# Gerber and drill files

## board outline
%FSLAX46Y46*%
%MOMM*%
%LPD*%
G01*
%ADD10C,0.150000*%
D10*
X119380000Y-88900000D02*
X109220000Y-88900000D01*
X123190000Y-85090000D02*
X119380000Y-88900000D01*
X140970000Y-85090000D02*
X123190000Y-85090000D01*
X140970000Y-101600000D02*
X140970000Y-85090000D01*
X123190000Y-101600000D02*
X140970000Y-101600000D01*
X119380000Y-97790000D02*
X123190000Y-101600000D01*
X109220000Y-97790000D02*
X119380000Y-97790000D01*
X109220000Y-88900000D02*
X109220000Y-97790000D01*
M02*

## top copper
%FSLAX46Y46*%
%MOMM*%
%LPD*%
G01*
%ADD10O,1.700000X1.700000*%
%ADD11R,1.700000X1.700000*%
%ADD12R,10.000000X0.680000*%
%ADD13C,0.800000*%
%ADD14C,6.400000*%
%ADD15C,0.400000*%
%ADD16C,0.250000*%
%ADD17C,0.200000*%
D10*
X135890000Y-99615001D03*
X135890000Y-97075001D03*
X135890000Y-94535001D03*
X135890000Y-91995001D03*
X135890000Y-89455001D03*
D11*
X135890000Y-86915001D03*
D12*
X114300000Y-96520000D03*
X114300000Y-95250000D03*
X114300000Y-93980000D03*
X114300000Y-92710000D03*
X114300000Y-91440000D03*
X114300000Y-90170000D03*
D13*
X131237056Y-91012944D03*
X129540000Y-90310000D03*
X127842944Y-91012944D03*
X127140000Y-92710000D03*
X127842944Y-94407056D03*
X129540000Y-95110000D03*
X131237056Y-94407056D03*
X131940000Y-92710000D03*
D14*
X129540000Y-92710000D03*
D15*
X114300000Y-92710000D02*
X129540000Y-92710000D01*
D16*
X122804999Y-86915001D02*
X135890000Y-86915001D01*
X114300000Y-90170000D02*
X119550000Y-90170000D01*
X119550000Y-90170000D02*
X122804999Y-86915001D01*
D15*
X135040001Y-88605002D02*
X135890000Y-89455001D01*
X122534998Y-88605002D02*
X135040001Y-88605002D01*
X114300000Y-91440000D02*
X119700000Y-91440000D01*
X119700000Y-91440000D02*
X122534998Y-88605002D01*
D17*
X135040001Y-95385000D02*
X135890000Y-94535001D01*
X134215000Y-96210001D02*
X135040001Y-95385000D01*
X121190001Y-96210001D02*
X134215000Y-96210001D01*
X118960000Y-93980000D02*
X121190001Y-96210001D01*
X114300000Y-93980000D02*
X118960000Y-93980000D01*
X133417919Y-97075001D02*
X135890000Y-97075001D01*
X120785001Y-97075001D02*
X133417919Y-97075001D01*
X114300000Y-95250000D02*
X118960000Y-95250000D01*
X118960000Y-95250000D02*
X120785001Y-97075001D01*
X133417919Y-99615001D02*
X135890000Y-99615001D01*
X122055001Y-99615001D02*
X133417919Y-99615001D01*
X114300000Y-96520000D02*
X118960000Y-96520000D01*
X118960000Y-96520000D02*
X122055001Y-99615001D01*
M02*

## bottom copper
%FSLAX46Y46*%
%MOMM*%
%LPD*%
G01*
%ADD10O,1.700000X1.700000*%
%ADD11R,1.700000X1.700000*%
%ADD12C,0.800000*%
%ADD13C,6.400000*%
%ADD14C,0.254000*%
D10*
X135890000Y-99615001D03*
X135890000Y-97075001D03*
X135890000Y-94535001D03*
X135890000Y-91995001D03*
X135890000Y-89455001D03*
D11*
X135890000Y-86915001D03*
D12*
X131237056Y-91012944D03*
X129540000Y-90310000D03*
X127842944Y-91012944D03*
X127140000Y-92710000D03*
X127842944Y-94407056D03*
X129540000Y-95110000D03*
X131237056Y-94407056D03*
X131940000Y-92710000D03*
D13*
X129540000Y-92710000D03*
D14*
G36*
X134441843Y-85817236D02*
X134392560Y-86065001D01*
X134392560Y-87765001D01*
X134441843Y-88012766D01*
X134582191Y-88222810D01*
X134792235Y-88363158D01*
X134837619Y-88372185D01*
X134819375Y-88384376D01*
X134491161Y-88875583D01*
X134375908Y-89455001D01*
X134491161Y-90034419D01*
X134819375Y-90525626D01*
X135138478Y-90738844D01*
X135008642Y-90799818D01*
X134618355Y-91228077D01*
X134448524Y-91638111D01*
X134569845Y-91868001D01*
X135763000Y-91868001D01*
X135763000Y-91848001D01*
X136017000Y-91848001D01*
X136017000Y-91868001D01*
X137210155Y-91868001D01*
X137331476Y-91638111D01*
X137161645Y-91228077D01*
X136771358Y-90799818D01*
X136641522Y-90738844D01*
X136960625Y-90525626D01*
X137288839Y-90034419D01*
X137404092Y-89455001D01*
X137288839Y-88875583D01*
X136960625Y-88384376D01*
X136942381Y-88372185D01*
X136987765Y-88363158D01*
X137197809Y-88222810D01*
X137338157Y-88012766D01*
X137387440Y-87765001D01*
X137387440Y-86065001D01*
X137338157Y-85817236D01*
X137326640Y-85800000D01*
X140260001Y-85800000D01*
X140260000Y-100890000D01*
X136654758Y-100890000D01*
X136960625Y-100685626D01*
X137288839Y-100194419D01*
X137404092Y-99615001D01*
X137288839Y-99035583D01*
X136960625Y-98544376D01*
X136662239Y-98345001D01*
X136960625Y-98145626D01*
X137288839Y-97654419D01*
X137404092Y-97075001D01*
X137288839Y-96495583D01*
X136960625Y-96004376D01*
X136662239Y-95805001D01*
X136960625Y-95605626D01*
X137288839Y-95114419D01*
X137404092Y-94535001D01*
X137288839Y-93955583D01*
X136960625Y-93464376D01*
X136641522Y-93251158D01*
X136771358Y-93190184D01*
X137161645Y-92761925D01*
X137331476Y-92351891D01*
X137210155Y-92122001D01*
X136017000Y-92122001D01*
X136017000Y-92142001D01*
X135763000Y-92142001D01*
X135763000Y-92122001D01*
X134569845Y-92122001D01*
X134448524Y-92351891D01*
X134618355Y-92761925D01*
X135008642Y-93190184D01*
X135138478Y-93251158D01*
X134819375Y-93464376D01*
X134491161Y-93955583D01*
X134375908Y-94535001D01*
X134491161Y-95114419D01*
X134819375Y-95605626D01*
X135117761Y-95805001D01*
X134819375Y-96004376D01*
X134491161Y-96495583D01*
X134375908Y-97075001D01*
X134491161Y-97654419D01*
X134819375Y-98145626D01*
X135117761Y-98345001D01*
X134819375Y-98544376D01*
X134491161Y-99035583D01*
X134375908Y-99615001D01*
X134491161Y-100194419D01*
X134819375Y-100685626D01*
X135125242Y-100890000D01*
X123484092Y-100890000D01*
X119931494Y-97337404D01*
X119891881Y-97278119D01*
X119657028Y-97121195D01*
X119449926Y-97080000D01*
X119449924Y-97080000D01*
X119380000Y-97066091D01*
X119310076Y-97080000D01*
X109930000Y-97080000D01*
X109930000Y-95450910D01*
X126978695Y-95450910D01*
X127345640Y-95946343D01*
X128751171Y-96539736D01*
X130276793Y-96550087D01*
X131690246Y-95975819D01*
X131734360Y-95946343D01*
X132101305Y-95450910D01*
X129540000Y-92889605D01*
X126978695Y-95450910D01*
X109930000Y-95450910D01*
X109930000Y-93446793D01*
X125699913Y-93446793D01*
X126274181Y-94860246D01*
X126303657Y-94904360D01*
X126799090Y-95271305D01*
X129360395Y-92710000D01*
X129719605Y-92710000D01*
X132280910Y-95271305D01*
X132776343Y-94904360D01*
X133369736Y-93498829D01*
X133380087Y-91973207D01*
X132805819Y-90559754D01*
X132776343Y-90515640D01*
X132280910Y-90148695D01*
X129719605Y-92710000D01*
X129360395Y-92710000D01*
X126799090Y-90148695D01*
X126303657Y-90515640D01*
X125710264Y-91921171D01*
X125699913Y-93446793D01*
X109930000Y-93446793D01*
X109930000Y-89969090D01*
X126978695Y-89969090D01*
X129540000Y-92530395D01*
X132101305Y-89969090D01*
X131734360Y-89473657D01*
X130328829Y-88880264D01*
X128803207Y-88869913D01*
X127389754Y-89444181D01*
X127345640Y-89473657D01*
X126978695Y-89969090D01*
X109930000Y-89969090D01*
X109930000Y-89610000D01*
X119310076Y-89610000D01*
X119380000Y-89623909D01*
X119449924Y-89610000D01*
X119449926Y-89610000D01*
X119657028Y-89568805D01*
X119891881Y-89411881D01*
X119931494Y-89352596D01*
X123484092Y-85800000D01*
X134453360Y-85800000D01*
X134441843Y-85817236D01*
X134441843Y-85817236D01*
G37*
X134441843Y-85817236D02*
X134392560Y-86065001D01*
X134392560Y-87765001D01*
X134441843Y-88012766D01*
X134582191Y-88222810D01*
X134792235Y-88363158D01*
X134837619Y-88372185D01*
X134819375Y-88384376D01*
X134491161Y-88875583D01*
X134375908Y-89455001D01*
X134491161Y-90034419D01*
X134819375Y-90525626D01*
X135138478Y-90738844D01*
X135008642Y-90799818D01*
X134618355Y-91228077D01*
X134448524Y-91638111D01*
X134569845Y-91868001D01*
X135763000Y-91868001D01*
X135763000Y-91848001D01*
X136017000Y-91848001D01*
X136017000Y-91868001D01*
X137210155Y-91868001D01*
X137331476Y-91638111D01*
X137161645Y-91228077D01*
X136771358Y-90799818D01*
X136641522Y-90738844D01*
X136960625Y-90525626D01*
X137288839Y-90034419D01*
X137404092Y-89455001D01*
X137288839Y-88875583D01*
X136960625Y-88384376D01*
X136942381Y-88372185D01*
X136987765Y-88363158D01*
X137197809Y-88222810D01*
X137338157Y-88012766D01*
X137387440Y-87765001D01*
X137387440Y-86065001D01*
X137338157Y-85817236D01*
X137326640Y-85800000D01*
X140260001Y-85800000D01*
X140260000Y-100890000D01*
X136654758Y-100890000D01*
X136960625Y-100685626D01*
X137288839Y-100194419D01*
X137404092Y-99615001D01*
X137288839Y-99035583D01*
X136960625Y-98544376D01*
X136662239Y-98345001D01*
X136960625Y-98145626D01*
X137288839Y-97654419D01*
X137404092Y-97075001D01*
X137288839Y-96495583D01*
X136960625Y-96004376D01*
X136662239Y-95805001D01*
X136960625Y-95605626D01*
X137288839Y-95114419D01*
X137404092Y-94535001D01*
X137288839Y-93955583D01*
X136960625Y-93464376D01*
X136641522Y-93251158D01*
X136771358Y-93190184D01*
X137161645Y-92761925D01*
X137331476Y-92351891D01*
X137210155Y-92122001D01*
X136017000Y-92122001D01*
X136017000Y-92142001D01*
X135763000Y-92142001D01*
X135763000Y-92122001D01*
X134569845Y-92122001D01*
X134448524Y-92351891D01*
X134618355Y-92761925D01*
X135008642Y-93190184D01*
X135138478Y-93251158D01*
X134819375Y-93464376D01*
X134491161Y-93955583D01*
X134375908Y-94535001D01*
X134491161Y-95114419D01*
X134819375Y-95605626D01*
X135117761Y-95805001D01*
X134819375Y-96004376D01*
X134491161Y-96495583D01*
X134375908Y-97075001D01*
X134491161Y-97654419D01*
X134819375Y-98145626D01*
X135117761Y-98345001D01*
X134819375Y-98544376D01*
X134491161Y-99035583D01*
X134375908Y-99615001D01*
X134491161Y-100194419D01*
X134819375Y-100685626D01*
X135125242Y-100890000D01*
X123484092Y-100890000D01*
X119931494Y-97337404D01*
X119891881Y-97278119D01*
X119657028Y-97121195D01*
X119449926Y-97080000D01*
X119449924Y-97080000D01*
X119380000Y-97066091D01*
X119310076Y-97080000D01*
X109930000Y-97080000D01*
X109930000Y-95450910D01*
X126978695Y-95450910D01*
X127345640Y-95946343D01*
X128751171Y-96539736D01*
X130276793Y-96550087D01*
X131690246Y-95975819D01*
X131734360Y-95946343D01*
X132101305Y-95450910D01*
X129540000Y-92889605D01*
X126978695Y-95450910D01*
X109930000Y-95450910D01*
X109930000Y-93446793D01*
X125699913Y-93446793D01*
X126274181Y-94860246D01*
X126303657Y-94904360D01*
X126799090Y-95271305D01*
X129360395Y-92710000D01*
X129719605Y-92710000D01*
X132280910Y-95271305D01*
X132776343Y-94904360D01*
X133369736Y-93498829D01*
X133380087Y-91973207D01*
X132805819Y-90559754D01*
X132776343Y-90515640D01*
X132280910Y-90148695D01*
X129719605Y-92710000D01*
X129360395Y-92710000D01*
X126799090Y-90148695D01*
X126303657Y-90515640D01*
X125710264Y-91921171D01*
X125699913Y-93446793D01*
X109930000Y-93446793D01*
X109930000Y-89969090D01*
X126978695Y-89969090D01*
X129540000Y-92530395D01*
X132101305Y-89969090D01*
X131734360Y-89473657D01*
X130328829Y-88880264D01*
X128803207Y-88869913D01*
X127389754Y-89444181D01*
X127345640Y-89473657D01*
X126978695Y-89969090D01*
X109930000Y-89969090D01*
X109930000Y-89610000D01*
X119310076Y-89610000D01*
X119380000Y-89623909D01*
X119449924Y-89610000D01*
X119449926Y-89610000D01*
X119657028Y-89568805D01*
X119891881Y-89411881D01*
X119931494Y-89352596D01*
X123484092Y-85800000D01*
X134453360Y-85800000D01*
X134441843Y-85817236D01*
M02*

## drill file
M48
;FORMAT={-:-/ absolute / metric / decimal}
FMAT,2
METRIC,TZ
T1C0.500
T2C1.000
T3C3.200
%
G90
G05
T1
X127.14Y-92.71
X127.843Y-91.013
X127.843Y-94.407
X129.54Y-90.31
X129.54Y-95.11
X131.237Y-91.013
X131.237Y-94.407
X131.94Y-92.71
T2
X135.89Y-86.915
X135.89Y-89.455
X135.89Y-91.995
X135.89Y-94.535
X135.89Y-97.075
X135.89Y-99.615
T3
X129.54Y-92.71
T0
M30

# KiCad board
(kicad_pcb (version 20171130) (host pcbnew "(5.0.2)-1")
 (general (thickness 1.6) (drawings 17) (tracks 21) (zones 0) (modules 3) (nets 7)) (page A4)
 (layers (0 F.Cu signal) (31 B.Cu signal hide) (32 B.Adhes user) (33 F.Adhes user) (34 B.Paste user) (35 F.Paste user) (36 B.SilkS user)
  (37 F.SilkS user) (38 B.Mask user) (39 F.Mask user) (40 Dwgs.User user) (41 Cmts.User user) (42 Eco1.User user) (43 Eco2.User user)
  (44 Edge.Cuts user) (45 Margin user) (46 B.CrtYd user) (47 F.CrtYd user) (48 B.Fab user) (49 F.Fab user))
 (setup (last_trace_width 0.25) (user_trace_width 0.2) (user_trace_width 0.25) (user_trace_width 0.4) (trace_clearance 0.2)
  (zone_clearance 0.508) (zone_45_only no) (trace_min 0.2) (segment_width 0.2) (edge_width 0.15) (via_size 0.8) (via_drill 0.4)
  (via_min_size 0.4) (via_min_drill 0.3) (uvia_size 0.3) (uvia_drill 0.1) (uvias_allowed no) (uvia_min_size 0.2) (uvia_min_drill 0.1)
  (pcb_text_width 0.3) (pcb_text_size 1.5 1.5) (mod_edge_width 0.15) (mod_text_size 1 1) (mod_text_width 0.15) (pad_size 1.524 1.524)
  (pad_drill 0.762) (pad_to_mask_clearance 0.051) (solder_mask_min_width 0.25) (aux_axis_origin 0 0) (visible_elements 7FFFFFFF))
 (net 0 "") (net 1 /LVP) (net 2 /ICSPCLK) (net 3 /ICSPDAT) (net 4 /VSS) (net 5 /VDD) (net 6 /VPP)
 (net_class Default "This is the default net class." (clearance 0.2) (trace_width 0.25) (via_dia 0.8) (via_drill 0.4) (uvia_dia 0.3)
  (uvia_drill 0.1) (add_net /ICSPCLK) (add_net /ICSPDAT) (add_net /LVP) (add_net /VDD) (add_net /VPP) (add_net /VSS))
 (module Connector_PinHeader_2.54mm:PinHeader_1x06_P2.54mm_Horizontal (layer F.Cu) (at 135.89 86.915001)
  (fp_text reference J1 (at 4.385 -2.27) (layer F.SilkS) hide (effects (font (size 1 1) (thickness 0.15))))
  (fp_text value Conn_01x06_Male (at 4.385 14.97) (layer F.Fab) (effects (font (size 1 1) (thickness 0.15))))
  (pad 6 thru_hole oval (at 0 12.7) (size 1.7 1.7) (drill 1) (layers *.Cu *.Mask) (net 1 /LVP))
  (pad 5 thru_hole oval (at 0 10.16) (size 1.7 1.7) (drill 1) (layers *.Cu *.Mask) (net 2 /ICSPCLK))
  (pad 4 thru_hole oval (at 0 7.62) (size 1.7 1.7) (drill 1) (layers *.Cu *.Mask) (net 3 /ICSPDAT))
  (pad 3 thru_hole oval (at 0 5.08) (size 1.7 1.7) (drill 1) (layers *.Cu *.Mask) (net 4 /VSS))
  (pad 2 thru_hole oval (at 0 2.54) (size 1.7 1.7) (drill 1) (layers *.Cu *.Mask) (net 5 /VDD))
  (pad 1 thru_hole rect (at 0 0) (size 1.7 1.7) (drill 1) (layers *.Cu *.Mask) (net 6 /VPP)))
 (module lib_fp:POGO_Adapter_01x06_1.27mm (layer F.Cu) (at 114.3 93.98 270)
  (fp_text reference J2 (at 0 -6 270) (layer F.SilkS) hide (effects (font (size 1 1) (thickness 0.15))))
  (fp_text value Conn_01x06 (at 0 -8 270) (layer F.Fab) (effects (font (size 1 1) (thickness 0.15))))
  (pad 6 smd rect (at 2.54 0 270) (size 0.68 10) (layers F.Cu F.Paste F.Mask) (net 1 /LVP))
  (pad 5 smd rect (at 1.27 0 270) (size 0.68 10) (layers F.Cu F.Paste F.Mask) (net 2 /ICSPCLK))
  (pad 4 smd rect (at 0 0 270) (size 0.68 10) (layers F.Cu F.Paste F.Mask) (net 3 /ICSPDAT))
  (pad 3 smd rect (at -1.27 0 270) (size 0.68 10) (layers F.Cu F.Paste F.Mask) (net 4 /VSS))
  (pad 2 smd rect (at -2.54 0 270) (size 0.68 10) (layers F.Cu F.Paste F.Mask) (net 5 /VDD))
  (pad 1 smd rect (at -3.81 0 270) (size 0.68 10) (layers F.Cu F.Paste F.Mask) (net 6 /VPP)))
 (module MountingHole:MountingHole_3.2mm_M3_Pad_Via (layer F.Cu) (at 129.54 92.71)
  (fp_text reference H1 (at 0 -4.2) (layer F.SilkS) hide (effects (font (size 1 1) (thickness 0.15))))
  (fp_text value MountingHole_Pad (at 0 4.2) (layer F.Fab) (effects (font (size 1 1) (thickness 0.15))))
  (pad 1 thru_hole circle (at 1.697056 -1.697056) (size 0.8 0.8) (drill 0.5) (layers *.Cu *.Mask) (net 4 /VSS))
  (pad 1 thru_hole circle (at 0 -2.4) (size 0.8 0.8) (drill 0.5) (layers *.Cu *.Mask) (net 4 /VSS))
  (pad 1 thru_hole circle (at -1.697056 -1.697056) (size 0.8 0.8) (drill 0.5) (layers *.Cu *.Mask) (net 4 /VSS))
  (pad 1 thru_hole circle (at -2.4 0) (size 0.8 0.8) (drill 0.5) (layers *.Cu *.Mask) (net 4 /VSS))
  (pad 1 thru_hole circle (at -1.697056 1.697056) (size 0.8 0.8) (drill 0.5) (layers *.Cu *.Mask) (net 4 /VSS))
  (pad 1 thru_hole circle (at 0 2.4) (size 0.8 0.8) (drill 0.5) (layers *.Cu *.Mask) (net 4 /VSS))
  (pad 1 thru_hole circle (at 1.697056 1.697056) (size 0.8 0.8) (drill 0.5) (layers *.Cu *.Mask) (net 4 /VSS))
  (pad 1 thru_hole circle (at 2.4 0) (size 0.8 0.8) (drill 0.5) (layers *.Cu *.Mask) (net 4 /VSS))
  (pad 1 thru_hole circle (at 0 0) (size 6.4 6.4) (drill 3.2) (layers *.Cu *.Mask) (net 4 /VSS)))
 (gr_line (start 119.38 88.9) (end 109.22 88.9) (layer Edge.Cuts) (width 0.15))
 (gr_line (start 123.19 85.09) (end 119.38 88.9) (layer Edge.Cuts) (width 0.15))
 (gr_line (start 140.97 85.09) (end 123.19 85.09) (layer Edge.Cuts) (width 0.15))
 (gr_line (start 140.97 101.6) (end 140.97 85.09) (layer Edge.Cuts) (width 0.15))
 (gr_line (start 123.19 101.6) (end 140.97 101.6) (layer Edge.Cuts) (width 0.15))
 (gr_line (start 119.38 97.79) (end 123.19 101.6) (layer Edge.Cuts) (width 0.15))
 (gr_line (start 109.22 97.79) (end 119.38 97.79) (layer Edge.Cuts) (width 0.15))
 (gr_line (start 109.22 88.9) (end 109.22 97.79) (layer Edge.Cuts) (width 0.15))
 (segment (start 114.3 92.71) (end 129.54 92.71) (width 0.4) (layer F.Cu) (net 4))
 (segment (start 122.804999 86.915001) (end 135.89 86.915001) (width 0.25) (layer F.Cu) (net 6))
 (segment (start 114.3 90.17) (end 119.55 90.17) (width 0.25) (layer F.Cu) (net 6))
 (segment (start 119.55 90.17) (end 122.804999 86.915001) (width 0.25) (layer F.Cu) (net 6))
 (segment (start 135.040001 88.605002) (end 135.89 89.455001) (width 0.4) (layer F.Cu) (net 5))
 (segment (start 122.534998 88.605002) (end 135.040001 88.605002) (width 0.4) (layer F.Cu) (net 5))
 (segment (start 114.3 91.44) (end 119.7 91.44) (width 0.4) (layer F.Cu) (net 5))
 (segment (start 119.7 91.44) (end 122.534998 88.605002) (width 0.4) (layer F.Cu) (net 5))
 (segment (start 135.040001 95.385) (end 135.89 94.535001) (width 0.2) (layer F.Cu) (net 3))
 (segment (start 134.215 96.210001) (end 135.040001 95.385) (width 0.2) (layer F.Cu) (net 3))
 (segment (start 121.190001 96.210001) (end 134.215 96.210001) (width 0.2) (layer F.Cu) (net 3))
 (segment (start 118.96 93.98) (end 121.190001 96.210001) (width 0.2) (layer F.Cu) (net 3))
 (segment (start 114.3 93.98) (end 118.96 93.98) (width 0.2) (layer F.Cu) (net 3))
 (segment (start 133.417919 97.075001) (end 135.89 97.075001) (width 0.2) (layer F.Cu) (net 2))
 (segment (start 120.785001 97.075001) (end 133.417919 97.075001) (width 0.2) (layer F.Cu) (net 2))
 (segment (start 114.3 95.25) (end 118.96 95.25) (width 0.2) (layer F.Cu) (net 2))
 (segment (start 118.96 95.25) (end 120.785001 97.075001) (width 0.2) (layer F.Cu) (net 2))
 (segment (start 133.417919 99.615001) (end 135.89 99.615001) (width 0.2) (layer F.Cu) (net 1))
 (segment (start 122.055001 99.615001) (end 133.417919 99.615001) (width 0.2) (layer F.Cu) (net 1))
 (segment (start 114.3 96.52) (end 118.96 96.52) (width 0.2) (layer F.Cu) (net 1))
 (segment (start 118.96 96.52) (end 122.055001 99.615001) (width 0.2) (layer F.Cu) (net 1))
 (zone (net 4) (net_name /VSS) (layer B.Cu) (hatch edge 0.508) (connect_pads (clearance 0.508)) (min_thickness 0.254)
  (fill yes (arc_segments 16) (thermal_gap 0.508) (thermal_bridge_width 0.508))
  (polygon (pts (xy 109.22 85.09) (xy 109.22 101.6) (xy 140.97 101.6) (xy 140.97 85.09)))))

